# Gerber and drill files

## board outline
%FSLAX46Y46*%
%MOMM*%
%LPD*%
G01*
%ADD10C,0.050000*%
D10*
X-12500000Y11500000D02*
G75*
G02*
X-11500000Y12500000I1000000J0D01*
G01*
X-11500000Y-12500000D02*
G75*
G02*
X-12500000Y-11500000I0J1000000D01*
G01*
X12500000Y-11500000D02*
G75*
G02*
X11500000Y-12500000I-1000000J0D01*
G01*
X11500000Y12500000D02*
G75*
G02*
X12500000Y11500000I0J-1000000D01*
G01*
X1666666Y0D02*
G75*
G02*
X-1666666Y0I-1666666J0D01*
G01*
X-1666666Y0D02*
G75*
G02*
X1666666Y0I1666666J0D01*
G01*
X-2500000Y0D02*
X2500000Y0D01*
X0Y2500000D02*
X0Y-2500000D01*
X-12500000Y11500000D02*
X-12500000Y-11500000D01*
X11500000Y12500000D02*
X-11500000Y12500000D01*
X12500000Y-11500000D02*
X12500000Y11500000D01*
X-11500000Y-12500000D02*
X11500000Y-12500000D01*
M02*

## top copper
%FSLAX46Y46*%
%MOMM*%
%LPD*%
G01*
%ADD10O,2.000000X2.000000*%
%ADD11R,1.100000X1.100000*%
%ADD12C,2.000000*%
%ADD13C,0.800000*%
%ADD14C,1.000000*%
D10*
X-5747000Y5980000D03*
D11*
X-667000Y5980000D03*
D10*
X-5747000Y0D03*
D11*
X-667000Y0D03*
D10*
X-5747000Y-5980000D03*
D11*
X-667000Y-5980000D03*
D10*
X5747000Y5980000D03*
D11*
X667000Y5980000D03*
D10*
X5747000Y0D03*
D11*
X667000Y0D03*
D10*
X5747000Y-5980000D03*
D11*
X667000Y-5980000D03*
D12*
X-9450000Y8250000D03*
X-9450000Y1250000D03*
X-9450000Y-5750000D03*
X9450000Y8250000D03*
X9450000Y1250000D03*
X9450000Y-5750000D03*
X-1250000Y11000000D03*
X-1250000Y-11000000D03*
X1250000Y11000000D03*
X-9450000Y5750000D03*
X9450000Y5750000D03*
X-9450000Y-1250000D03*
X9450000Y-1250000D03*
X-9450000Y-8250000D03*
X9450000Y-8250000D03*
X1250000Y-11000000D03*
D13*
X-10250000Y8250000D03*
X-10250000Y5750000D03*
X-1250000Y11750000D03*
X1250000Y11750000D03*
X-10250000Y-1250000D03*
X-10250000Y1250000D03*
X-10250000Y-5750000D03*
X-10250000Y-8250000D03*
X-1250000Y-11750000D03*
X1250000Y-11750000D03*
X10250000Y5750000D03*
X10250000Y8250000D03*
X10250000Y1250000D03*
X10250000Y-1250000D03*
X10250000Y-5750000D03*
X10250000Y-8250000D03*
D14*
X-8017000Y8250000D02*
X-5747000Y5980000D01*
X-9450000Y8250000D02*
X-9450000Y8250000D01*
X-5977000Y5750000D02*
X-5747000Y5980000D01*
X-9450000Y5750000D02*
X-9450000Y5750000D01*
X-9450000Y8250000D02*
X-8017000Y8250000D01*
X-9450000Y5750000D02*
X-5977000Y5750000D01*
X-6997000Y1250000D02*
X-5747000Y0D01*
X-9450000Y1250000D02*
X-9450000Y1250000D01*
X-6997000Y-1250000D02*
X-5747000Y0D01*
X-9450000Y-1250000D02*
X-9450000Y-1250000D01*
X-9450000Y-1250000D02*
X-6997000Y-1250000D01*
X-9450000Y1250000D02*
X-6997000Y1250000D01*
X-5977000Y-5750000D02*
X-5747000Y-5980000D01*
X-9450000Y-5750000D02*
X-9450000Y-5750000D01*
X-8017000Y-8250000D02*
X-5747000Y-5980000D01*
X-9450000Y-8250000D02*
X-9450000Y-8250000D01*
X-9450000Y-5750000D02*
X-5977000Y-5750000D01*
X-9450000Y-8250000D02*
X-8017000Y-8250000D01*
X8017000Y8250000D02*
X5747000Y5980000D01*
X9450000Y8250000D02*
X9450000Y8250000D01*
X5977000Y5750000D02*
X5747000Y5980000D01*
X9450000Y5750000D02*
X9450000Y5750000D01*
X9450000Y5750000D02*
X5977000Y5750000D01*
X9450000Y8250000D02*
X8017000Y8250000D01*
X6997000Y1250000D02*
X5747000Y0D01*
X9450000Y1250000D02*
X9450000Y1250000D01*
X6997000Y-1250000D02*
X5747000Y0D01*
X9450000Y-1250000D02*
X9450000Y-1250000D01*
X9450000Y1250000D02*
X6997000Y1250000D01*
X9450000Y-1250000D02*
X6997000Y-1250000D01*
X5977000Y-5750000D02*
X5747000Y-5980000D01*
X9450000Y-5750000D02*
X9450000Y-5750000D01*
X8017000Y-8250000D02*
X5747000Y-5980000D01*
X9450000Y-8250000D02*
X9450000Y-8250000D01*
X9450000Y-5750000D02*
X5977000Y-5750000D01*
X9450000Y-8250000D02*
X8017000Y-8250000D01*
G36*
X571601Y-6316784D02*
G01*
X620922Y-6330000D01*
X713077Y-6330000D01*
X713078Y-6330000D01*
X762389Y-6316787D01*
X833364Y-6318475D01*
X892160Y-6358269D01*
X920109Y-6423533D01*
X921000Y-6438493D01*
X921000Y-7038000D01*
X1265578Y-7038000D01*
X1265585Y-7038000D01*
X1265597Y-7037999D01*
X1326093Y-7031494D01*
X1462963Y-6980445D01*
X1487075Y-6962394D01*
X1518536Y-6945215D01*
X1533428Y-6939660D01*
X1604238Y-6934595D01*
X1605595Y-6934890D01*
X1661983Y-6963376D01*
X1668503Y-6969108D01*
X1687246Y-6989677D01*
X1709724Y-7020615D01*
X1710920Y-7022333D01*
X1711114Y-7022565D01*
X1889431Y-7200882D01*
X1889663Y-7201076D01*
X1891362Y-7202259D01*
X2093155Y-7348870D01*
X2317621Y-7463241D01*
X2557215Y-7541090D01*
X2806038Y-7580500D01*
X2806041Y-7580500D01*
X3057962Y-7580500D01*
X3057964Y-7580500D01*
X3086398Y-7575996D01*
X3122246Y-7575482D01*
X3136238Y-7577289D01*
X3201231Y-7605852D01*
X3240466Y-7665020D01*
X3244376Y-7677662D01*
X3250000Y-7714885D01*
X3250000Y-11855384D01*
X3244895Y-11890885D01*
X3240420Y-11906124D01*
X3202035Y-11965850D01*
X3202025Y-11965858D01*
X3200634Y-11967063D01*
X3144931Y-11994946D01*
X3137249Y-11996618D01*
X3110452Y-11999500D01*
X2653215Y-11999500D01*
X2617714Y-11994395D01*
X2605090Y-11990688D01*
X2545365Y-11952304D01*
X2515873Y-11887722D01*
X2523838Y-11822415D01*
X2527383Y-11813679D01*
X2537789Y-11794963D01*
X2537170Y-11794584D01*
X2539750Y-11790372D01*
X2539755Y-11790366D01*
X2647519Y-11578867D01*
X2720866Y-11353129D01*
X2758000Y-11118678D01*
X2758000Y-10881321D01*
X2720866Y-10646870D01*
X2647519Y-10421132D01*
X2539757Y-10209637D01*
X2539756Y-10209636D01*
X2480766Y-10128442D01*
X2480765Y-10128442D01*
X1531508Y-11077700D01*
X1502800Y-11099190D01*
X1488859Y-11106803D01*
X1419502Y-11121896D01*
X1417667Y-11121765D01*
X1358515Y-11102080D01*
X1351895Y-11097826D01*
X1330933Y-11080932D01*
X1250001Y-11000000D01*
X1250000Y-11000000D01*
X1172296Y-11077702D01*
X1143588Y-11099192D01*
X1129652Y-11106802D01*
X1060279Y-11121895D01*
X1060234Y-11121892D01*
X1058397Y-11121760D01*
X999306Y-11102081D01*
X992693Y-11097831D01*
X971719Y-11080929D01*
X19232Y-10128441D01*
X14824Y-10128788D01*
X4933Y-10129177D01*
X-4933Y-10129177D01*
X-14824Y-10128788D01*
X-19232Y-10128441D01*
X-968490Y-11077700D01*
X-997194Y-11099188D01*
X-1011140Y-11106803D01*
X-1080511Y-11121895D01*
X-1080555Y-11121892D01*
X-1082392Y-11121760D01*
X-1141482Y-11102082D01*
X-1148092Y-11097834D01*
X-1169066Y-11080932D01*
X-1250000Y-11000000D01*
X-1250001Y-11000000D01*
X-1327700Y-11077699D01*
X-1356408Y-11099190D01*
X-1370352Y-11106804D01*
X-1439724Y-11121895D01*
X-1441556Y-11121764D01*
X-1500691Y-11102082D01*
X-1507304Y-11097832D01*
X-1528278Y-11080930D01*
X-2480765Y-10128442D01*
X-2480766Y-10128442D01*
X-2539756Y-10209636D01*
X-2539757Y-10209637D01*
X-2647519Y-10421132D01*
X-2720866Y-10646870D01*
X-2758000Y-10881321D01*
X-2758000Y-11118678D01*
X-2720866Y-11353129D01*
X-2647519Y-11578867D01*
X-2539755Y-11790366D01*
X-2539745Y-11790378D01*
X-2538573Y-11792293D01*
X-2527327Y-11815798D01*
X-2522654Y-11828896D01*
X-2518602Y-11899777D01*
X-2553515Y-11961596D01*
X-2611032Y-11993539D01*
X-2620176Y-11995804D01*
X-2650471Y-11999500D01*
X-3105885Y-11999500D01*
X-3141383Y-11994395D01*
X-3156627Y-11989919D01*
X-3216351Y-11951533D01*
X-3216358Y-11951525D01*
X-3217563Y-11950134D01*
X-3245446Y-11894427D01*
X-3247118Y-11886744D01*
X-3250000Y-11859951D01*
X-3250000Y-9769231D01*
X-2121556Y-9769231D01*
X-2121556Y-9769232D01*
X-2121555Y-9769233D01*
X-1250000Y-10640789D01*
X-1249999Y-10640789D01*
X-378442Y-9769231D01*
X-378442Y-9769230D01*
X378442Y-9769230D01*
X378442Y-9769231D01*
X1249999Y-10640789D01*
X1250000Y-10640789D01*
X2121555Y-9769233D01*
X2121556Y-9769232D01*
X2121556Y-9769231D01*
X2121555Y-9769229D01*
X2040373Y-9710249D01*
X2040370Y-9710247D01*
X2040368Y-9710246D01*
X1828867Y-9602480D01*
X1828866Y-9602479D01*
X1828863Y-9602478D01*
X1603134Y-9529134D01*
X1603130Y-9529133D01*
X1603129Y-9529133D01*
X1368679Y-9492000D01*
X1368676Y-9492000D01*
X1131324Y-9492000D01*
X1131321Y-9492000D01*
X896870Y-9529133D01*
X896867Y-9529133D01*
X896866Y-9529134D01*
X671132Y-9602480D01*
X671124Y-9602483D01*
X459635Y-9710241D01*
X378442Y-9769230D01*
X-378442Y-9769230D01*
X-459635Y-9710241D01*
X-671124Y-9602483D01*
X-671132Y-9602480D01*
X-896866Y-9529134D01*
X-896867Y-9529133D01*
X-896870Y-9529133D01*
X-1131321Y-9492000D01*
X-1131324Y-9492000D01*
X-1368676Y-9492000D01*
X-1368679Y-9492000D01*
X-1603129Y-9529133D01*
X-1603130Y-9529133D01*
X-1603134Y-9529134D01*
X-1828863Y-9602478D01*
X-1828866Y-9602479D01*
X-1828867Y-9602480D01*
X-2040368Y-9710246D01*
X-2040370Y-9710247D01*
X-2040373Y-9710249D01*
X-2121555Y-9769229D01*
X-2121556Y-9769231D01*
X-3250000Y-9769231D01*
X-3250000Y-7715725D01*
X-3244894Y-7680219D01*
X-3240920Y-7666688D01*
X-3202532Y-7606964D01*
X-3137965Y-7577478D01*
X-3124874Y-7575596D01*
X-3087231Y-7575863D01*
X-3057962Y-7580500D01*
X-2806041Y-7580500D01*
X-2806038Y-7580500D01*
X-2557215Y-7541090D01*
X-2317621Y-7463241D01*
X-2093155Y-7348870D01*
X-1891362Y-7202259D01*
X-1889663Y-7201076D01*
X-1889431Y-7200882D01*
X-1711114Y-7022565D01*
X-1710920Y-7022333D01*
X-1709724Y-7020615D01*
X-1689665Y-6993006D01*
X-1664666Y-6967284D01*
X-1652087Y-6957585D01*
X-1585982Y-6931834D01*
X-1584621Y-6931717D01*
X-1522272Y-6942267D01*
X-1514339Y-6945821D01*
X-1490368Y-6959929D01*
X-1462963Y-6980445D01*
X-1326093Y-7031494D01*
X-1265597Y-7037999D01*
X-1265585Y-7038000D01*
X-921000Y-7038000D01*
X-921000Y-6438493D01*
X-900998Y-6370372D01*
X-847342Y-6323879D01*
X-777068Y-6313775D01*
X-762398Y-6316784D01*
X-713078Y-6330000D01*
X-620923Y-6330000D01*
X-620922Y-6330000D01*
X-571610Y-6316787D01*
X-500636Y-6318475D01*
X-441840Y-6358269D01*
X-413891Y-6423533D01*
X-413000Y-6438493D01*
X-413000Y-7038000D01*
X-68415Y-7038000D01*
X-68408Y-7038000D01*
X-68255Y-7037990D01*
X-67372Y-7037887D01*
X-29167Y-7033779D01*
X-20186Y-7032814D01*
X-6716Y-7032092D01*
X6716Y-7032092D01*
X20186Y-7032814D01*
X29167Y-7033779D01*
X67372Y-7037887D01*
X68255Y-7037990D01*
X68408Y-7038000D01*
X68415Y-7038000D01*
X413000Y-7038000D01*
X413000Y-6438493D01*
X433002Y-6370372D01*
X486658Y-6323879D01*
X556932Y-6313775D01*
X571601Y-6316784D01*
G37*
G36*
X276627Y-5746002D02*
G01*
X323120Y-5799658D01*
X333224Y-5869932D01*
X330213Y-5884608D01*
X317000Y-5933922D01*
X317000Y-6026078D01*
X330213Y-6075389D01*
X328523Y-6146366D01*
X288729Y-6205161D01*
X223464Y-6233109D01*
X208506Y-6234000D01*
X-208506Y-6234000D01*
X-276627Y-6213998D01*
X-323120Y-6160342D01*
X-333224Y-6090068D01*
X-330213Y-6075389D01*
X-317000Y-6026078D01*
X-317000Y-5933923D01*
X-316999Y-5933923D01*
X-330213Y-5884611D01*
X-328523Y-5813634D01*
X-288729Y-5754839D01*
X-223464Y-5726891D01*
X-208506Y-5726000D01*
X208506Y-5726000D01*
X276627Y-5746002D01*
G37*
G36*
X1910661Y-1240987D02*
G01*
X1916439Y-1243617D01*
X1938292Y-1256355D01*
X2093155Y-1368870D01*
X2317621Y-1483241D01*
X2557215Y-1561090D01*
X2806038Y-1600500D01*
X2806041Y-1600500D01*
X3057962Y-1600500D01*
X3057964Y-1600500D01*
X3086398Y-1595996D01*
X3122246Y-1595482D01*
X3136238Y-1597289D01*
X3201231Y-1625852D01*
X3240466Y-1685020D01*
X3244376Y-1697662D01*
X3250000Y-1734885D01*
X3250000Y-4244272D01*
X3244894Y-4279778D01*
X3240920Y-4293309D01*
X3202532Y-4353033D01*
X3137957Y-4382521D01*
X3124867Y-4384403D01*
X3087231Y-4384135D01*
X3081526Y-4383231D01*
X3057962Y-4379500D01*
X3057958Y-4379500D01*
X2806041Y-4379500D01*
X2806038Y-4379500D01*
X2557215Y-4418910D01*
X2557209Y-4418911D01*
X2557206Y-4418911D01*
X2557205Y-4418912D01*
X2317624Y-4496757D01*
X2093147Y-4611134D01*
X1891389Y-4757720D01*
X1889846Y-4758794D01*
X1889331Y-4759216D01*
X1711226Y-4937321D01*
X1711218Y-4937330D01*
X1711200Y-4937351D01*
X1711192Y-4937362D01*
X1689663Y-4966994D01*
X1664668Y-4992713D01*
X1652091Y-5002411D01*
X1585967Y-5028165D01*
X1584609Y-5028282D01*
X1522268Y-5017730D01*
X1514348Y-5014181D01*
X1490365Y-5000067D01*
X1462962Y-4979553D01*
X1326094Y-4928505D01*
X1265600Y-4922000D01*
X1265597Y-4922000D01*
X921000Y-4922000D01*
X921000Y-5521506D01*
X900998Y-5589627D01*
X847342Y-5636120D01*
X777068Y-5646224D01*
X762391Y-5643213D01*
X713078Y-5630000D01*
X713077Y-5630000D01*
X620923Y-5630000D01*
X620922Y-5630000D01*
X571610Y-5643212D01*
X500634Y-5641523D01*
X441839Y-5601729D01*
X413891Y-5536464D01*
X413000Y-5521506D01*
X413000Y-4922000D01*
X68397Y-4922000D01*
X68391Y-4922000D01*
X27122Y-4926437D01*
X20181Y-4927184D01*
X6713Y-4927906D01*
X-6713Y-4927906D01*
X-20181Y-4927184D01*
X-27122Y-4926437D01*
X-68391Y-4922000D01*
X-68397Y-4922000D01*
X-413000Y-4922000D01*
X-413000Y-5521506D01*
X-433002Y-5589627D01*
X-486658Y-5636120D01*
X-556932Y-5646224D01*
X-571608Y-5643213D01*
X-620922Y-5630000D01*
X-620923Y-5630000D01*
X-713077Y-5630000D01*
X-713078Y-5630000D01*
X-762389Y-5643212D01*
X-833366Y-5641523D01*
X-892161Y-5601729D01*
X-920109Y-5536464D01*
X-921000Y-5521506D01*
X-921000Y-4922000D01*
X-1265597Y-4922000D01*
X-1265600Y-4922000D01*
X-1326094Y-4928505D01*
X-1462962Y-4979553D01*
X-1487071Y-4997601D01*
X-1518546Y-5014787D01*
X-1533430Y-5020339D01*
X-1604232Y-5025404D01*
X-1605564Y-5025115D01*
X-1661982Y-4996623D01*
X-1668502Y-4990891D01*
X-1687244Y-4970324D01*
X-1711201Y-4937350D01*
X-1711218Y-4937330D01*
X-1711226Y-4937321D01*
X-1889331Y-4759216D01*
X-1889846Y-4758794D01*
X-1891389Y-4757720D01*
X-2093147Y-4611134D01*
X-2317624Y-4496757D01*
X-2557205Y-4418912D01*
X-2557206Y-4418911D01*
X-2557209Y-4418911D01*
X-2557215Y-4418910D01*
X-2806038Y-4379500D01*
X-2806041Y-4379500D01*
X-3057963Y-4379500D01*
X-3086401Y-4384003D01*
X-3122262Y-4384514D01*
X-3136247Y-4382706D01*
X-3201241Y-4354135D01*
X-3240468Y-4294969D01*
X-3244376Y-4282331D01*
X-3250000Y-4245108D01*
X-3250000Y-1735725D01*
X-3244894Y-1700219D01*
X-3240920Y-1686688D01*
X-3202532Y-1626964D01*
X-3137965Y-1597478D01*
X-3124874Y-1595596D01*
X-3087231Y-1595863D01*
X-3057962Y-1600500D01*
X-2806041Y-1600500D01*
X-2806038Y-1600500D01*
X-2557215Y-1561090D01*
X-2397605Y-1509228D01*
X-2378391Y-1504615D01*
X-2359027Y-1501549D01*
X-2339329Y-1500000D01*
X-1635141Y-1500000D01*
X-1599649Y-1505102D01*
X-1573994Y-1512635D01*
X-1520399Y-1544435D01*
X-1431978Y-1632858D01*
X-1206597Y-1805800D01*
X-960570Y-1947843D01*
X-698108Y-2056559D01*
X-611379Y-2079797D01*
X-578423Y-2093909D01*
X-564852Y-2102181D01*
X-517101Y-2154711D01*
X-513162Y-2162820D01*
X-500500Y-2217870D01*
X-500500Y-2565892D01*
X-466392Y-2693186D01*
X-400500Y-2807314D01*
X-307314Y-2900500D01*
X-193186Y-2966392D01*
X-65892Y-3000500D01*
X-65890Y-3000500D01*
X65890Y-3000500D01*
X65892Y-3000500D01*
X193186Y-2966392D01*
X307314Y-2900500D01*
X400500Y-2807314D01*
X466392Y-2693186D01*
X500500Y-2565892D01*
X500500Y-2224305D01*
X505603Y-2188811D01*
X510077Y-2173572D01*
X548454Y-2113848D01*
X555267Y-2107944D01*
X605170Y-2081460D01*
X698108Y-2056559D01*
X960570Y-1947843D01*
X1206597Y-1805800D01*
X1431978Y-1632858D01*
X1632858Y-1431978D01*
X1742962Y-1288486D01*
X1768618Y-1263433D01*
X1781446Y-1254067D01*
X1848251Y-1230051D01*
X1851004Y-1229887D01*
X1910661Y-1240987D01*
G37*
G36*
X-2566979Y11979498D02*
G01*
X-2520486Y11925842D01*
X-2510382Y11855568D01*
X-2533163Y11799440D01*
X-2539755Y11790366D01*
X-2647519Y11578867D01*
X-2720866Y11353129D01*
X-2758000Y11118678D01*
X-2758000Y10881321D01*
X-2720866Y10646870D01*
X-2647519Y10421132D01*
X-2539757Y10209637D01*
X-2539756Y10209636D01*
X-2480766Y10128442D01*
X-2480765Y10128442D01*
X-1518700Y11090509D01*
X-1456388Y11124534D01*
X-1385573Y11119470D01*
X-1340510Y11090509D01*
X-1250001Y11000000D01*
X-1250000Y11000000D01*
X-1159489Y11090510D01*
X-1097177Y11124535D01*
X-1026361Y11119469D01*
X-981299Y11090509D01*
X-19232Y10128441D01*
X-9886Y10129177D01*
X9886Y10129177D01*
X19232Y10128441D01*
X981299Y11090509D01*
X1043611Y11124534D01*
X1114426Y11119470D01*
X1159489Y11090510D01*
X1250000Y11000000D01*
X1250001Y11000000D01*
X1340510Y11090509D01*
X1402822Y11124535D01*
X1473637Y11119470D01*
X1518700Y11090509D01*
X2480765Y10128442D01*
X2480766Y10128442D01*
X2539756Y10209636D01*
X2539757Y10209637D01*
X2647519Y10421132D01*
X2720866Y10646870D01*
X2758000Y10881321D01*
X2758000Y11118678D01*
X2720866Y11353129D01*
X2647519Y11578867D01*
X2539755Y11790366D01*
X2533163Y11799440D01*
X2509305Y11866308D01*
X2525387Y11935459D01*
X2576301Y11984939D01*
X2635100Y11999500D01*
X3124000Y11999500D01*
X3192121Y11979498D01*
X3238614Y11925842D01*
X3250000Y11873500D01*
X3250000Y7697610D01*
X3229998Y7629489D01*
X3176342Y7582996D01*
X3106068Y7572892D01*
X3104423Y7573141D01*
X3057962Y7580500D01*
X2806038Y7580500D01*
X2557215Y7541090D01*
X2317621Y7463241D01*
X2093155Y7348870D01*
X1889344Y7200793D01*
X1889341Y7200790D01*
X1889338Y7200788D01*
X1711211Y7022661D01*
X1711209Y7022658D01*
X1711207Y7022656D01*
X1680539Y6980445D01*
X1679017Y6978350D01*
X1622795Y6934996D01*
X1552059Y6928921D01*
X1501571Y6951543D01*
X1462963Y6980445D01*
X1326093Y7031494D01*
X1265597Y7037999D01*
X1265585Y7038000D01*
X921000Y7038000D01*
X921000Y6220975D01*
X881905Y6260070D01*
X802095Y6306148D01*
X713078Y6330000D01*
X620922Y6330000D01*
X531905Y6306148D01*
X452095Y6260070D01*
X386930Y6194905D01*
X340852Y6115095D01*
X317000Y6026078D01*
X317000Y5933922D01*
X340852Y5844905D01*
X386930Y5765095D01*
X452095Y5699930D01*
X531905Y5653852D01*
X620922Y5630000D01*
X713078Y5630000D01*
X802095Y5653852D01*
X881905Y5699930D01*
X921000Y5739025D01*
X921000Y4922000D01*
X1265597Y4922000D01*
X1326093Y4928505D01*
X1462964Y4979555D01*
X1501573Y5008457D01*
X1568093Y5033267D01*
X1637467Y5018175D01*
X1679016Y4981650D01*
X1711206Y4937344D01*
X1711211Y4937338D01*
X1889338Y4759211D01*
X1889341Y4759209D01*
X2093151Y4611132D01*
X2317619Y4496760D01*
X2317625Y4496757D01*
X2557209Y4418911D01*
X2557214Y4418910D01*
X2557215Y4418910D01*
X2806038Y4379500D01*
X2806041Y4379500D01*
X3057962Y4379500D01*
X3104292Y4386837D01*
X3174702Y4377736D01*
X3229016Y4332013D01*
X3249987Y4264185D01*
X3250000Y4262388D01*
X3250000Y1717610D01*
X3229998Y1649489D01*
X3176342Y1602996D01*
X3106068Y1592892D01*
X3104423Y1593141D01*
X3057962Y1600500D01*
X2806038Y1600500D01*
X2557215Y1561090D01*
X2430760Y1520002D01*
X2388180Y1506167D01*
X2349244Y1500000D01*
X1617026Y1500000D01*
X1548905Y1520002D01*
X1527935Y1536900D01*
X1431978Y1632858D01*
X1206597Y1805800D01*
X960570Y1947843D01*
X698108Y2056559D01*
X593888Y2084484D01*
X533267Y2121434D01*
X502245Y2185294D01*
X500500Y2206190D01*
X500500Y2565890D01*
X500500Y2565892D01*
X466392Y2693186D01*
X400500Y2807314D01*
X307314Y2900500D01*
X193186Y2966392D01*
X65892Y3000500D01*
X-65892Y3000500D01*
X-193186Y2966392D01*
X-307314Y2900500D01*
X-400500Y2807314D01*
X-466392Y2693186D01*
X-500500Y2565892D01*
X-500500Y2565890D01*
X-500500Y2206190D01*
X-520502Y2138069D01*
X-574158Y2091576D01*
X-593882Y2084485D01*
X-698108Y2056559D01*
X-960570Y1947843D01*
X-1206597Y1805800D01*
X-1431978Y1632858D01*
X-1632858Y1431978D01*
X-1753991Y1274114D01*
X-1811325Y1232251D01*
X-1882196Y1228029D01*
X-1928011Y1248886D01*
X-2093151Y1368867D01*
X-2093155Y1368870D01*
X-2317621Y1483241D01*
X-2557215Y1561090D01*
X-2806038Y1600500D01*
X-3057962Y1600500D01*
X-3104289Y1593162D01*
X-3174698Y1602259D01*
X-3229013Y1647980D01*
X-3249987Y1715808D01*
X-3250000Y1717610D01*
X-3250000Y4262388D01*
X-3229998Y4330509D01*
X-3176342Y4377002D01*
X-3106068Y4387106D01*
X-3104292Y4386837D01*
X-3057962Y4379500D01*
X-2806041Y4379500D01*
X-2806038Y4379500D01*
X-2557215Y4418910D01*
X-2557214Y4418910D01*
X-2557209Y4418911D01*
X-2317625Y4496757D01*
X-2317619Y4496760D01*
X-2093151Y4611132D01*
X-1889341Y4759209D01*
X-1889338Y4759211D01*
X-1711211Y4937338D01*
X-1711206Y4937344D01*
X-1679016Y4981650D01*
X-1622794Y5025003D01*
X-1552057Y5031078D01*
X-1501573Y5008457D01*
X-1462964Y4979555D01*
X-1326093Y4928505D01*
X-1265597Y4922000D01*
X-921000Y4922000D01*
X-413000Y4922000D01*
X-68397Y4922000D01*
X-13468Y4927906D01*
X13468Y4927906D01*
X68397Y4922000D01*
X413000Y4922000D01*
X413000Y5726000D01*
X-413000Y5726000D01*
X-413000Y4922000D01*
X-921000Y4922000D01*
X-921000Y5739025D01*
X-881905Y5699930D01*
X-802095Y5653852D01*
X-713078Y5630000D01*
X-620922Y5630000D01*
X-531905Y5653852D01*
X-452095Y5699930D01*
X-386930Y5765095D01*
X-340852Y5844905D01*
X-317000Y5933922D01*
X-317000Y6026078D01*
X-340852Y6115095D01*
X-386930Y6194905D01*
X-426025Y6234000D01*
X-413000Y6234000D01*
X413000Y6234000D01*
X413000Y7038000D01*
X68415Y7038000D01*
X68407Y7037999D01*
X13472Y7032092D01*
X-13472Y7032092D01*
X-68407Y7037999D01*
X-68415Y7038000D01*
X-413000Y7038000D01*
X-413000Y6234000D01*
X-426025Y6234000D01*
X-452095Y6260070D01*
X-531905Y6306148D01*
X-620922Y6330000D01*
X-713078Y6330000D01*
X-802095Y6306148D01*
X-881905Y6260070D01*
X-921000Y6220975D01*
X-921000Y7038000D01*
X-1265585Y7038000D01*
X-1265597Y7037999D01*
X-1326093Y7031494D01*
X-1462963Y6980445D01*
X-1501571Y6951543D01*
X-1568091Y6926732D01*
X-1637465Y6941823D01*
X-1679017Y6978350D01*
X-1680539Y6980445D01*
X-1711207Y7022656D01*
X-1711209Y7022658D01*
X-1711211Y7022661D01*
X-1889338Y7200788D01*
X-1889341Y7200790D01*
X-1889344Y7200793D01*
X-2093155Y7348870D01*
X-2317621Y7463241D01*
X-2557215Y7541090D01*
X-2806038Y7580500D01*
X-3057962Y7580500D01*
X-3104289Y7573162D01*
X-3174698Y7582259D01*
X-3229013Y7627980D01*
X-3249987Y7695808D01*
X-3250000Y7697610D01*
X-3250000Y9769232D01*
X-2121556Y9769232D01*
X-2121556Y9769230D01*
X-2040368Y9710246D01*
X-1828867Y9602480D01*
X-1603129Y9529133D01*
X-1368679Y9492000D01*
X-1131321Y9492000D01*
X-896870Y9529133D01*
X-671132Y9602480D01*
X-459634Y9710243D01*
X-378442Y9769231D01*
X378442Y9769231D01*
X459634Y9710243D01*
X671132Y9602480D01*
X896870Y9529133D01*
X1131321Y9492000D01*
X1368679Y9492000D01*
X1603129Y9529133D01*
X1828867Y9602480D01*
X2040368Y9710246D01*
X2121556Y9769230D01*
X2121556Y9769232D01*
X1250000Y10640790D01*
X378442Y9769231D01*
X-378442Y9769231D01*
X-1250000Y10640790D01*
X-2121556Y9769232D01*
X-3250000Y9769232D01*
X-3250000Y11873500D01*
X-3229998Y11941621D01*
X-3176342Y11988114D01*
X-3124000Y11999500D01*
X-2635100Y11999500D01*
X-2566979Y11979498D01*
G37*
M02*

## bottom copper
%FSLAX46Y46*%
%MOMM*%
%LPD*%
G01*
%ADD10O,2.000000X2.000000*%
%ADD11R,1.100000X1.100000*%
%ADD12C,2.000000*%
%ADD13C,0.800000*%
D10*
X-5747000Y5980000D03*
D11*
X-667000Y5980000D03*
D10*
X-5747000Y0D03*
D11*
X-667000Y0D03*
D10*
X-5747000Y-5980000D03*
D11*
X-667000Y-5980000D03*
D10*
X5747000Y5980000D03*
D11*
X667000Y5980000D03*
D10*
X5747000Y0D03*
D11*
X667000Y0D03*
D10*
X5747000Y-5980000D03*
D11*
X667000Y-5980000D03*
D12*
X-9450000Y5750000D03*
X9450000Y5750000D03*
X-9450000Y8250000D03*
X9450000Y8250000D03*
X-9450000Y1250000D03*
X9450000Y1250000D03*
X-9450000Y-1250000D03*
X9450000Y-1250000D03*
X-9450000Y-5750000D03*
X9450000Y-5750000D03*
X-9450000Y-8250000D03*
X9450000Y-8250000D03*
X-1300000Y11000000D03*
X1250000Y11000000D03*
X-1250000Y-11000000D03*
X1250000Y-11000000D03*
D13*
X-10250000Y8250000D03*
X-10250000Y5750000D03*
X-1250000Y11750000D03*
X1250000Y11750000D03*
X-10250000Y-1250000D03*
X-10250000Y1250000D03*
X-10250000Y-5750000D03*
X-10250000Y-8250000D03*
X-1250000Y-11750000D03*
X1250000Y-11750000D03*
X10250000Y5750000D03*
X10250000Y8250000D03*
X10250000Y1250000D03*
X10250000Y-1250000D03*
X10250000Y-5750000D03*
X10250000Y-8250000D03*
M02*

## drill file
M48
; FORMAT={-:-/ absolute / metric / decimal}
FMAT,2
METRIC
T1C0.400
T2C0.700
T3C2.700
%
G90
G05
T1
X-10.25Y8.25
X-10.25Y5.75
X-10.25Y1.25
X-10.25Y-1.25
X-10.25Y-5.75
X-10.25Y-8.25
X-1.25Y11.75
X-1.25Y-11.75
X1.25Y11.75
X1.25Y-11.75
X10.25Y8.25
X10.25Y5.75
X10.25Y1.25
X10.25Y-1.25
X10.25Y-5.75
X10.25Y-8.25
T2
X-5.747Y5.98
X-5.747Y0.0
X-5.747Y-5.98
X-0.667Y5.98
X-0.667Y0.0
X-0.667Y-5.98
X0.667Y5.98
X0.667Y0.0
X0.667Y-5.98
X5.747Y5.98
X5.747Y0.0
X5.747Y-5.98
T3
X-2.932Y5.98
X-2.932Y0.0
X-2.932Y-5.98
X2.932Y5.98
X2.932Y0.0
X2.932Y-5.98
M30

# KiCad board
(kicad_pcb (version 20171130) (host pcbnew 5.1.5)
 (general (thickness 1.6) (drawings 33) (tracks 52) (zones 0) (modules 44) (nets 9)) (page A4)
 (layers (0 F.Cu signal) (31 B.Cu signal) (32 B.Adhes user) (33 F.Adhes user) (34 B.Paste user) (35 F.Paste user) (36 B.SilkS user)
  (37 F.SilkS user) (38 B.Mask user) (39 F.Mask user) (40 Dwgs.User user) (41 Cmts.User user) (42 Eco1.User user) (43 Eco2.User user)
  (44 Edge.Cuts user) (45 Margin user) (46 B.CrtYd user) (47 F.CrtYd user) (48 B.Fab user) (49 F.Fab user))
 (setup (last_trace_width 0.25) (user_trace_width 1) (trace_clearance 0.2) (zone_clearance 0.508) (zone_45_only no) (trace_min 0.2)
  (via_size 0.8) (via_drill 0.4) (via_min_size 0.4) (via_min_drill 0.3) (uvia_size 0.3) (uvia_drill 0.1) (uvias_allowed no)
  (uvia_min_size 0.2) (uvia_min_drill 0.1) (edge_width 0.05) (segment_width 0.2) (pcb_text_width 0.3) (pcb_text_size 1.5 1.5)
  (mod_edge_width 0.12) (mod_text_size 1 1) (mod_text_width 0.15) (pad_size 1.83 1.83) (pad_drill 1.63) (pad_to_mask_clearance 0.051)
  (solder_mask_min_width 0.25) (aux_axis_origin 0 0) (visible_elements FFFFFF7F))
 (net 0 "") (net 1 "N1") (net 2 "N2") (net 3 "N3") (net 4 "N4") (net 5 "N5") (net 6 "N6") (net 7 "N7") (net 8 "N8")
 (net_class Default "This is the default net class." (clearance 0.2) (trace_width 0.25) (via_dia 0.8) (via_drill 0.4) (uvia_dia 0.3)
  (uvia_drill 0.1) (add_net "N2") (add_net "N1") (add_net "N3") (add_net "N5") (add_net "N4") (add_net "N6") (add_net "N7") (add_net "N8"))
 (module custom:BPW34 (layer F.Cu) (at -2.932 -5.98 180)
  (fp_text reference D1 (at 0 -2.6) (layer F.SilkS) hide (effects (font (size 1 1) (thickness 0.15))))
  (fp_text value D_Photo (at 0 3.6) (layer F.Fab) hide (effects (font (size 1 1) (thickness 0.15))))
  (pad 2 thru_hole oval (at 2.815 0 180) (size 2 2) (drill 0.7) (layers *.Cu *.Mask) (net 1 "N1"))
  (pad 1 thru_hole rect (at -2.265 0 180) (size 1.1 1.1) (drill 0.7) (layers *.Cu *.Mask) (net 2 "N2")))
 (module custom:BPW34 (layer F.Cu) (at -2.932 0 180)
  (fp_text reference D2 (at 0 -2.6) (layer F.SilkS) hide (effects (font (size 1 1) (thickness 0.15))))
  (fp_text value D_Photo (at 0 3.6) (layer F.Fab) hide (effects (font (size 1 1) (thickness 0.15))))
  (pad 2 thru_hole oval (at 2.815 0 180) (size 2 2) (drill 0.7) (layers *.Cu *.Mask) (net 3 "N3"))
  (pad 1 thru_hole rect (at -2.265 0 180) (size 1.1 1.1) (drill 0.7) (layers *.Cu *.Mask) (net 2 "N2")))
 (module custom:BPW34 (layer F.Cu) (at -2.932 5.98 180)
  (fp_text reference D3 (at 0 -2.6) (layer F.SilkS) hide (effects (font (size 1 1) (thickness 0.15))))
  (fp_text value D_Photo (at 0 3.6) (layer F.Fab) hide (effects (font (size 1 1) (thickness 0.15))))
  (pad 2 thru_hole oval (at 2.815 0 180) (size 2 2) (drill 0.7) (layers *.Cu *.Mask) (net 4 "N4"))
  (pad 1 thru_hole rect (at -2.265 0 180) (size 1.1 1.1) (drill 0.7) (layers *.Cu *.Mask) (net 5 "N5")))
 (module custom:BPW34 (layer F.Cu) (at 2.932 -5.98)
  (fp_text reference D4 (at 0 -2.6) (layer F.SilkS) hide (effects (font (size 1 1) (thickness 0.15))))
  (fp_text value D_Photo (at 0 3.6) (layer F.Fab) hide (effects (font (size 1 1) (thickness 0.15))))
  (pad 2 thru_hole oval (at 2.815 0) (size 2 2) (drill 0.7) (layers *.Cu *.Mask) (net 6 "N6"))
  (pad 1 thru_hole rect (at -2.265 0) (size 1.1 1.1) (drill 0.7) (layers *.Cu *.Mask) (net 2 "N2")))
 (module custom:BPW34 (layer F.Cu) (at 2.932 0)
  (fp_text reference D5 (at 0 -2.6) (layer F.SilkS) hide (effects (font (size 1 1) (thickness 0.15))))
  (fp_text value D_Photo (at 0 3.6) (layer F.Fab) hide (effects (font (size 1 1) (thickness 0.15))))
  (pad 2 thru_hole oval (at 2.815 0) (size 2 2) (drill 0.7) (layers *.Cu *.Mask) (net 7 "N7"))
  (pad 1 thru_hole rect (at -2.265 0) (size 1.1 1.1) (drill 0.7) (layers *.Cu *.Mask) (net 5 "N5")))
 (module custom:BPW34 (layer F.Cu) (at 2.932 5.98)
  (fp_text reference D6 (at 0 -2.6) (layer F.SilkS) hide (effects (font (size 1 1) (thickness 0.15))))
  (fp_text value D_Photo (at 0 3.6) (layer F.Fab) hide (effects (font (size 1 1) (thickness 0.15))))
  (pad 2 thru_hole oval (at 2.815 0) (size 2 2) (drill 0.7) (layers *.Cu *.Mask) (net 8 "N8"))
  (pad 1 thru_hole rect (at -2.265 0) (size 1.1 1.1) (drill 0.7) (layers *.Cu *.Mask) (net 5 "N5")))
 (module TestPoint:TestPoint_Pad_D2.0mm (layer F.Cu) (at -9.45 -8.25)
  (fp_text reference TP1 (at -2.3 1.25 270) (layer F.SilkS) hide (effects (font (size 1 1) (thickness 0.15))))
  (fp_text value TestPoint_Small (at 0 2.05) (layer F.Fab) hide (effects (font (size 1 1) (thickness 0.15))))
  (pad 1 smd circle (at 0 0) (size 2 2) (layers F.Cu F.Mask) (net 1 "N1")))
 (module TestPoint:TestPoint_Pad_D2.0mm (layer F.Cu) (at -9.45 -1.25)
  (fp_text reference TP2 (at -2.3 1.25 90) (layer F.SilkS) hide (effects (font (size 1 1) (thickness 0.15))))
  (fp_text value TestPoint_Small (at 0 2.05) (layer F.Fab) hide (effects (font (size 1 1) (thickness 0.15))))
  (pad 1 smd circle (at 0 0) (size 2 2) (layers F.Cu F.Mask) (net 3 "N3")))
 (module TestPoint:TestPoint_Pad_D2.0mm (layer F.Cu) (at -9.45 5.75)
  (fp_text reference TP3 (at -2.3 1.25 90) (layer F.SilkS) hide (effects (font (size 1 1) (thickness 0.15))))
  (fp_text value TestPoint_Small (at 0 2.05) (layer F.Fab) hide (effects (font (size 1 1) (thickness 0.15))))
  (pad 1 smd circle (at 0 0) (size 2 2) (layers F.Cu F.Mask) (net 4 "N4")))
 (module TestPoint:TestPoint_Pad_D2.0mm (layer F.Cu) (at 9.45 -8.25)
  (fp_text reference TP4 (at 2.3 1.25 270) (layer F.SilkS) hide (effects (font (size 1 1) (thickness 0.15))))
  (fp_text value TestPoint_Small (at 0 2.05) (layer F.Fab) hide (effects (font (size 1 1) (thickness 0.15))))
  (pad 1 smd circle (at 0 0) (size 2 2) (layers F.Cu F.Mask) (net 6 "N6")))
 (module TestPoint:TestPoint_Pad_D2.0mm (layer F.Cu) (at 9.45 -1.25)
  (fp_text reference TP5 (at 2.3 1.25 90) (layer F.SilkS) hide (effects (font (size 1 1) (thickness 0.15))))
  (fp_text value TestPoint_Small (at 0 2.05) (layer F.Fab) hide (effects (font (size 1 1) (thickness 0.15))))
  (pad 1 smd circle (at 0 0) (size 2 2) (layers F.Cu F.Mask) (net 7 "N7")))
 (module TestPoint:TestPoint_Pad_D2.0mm (layer F.Cu) (at 9.45 5.75)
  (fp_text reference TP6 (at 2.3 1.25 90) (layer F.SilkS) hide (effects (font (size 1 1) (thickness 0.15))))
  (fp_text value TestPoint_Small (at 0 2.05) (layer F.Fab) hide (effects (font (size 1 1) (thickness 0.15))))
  (pad 1 smd circle (at 0 0) (size 2 2) (layers F.Cu F.Mask) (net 8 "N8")))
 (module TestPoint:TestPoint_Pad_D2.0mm (layer F.Cu) (at -1.25 -11)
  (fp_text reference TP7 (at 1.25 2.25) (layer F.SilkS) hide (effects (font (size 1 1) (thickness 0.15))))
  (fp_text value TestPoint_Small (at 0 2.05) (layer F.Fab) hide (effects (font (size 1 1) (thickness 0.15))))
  (pad 1 smd circle (at 0 0) (size 2 2) (layers F.Cu F.Mask) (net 2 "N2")))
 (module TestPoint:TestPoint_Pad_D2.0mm (layer F.Cu) (at -1.25 11)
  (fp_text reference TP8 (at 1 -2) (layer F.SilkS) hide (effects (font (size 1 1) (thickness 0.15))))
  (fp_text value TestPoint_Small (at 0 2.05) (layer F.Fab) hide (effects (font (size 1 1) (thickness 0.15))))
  (pad 1 smd circle (at 0 0) (size 2 2) (layers F.Cu F.Mask) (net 5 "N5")))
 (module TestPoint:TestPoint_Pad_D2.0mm (layer F.Cu) (at 1.25 -11)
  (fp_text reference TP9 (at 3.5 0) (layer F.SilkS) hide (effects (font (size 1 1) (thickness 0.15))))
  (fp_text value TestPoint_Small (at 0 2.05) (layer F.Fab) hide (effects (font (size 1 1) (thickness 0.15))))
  (pad 1 smd circle (at 0 0) (size 2 2) (layers F.Cu F.Mask) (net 2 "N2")))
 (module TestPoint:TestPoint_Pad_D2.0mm (layer F.Cu) (at -9.45 -5.75)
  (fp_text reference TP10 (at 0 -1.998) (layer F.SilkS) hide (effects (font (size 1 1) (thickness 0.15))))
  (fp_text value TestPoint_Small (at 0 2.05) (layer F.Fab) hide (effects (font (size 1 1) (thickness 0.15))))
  (pad 1 smd circle (at 0 0) (size 2 2) (layers F.Cu F.Mask) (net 1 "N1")))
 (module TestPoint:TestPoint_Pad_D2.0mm (layer F.Cu) (at 9.45 -5.75)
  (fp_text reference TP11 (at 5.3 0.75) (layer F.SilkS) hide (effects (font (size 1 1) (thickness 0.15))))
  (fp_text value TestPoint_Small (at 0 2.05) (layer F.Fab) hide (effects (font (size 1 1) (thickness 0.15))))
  (pad 1 smd circle (at 0 0) (size 2 2) (layers F.Cu F.Mask) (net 6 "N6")))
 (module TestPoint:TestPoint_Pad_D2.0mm (layer F.Cu) (at -9.45 1.25)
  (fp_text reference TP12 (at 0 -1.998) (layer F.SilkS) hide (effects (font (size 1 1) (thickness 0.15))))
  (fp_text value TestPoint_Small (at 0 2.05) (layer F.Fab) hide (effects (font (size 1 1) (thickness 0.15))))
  (pad 1 smd circle (at 0 0) (size 2 2) (layers F.Cu F.Mask) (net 3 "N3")))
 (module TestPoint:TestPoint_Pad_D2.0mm (layer F.Cu) (at 9.45 1.25)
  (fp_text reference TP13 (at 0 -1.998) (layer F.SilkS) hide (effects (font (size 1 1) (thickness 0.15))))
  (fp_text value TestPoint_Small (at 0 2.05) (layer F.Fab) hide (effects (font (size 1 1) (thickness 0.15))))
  (pad 1 smd circle (at 0 0) (size 2 2) (layers F.Cu F.Mask) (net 7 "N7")))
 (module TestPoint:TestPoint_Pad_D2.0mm (layer F.Cu) (at -9.45 8.25)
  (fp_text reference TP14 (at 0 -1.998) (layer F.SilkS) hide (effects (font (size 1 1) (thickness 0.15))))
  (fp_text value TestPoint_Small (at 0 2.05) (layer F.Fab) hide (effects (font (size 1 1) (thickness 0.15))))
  (pad 1 smd circle (at 0 0) (size 2 2) (layers F.Cu F.Mask) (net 4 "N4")))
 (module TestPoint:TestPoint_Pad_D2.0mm (layer F.Cu) (at 9.45 8.25)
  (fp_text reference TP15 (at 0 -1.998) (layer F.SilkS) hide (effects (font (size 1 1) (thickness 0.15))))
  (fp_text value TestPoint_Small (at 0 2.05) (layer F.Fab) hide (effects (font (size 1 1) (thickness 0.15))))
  (pad 1 smd circle (at 0 0) (size 2 2) (layers F.Cu F.Mask) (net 8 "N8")))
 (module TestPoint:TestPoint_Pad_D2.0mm (layer F.Cu) (at 1.25 11)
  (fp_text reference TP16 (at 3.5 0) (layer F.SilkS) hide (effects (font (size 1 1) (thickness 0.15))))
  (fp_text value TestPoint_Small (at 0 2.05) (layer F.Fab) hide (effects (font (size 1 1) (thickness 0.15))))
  (pad 1 smd circle (at 0 0) (size 2 2) (layers F.Cu F.Mask) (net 5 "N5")))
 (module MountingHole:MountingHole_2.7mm (layer F.Cu) (at -2.932 -5.98)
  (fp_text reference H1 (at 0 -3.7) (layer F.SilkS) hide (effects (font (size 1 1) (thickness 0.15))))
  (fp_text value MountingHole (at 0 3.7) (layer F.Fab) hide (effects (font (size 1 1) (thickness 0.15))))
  (pad 1 np_thru_hole circle (at 0 0) (size 2.7 2.7) (drill 2.7) (layers *.Cu *.Mask)))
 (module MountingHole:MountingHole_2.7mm (layer F.Cu) (at -2.932 0)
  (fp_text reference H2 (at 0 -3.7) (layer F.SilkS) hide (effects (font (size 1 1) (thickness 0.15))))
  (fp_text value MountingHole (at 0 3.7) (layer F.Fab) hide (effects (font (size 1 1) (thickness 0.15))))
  (pad 1 np_thru_hole circle (at 0 0) (size 2.7 2.7) (drill 2.7) (layers *.Cu *.Mask)))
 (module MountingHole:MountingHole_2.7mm (layer F.Cu) (at -2.932 5.98)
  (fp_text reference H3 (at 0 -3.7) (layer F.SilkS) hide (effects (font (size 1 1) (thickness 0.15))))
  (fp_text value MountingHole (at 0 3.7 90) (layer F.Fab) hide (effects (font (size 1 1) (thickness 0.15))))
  (pad 1 np_thru_hole circle (at 0 0) (size 2.7 2.7) (drill 2.7) (layers *.Cu *.Mask)))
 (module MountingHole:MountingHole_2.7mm (layer F.Cu) (at 2.932 -5.98)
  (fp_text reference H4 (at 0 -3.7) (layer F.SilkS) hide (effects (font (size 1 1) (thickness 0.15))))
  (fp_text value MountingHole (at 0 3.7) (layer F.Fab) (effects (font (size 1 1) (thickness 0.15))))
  (pad 1 np_thru_hole circle (at 0 0) (size 2.7 2.7) (drill 2.7) (layers *.Cu *.Mask)))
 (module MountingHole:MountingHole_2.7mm (layer F.Cu) (at 2.932 0)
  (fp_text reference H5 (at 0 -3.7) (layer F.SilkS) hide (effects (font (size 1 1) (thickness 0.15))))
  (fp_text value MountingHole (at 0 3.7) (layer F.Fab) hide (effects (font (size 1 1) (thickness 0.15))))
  (pad 1 np_thru_hole circle (at 0 0) (size 2.7 2.7) (drill 2.7) (layers *.Cu *.Mask)))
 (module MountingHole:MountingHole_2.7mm (layer F.Cu) (at 2.932 5.98)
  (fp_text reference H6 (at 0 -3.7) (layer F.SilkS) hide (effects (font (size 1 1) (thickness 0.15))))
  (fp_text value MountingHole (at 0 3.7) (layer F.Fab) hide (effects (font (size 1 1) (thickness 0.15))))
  (pad 1 np_thru_hole circle (at 0 0) (size 2.7 2.7) (drill 2.7) (layers *.Cu *.Mask)))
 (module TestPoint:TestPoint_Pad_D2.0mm (layer B.Cu) (at -9.45 -5.75)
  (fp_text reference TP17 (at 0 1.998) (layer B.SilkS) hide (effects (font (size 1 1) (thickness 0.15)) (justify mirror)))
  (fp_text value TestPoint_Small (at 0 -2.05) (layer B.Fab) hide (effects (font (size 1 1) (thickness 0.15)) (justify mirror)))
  (pad 1 smd circle (at 0 0) (size 2 2) (layers B.Cu B.Mask) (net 1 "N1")))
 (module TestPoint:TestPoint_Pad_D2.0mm (layer B.Cu) (at 9.45 -5.75)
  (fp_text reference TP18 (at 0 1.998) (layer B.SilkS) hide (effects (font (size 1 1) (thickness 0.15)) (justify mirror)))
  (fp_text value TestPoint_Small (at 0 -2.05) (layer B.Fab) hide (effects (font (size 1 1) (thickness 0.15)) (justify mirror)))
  (pad 1 smd circle (at 0 0) (size 2 2) (layers B.Cu B.Mask) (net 6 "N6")))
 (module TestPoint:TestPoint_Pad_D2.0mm (layer B.Cu) (at -9.45 -8.25)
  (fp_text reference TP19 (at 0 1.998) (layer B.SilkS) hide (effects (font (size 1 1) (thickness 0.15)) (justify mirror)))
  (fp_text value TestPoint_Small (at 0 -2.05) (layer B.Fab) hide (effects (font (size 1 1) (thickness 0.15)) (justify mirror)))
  (pad 1 smd circle (at 0 0) (size 2 2) (layers B.Cu B.Mask) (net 1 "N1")))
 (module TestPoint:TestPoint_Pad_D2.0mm (layer B.Cu) (at 9.45 -8.25)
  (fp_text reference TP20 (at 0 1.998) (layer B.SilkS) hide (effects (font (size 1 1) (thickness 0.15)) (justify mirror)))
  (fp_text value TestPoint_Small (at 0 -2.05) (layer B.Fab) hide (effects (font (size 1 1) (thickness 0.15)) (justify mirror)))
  (pad 1 smd circle (at 0 0) (size 2 2) (layers B.Cu B.Mask) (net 6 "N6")))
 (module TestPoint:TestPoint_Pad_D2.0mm (layer B.Cu) (at -9.45 -1.25)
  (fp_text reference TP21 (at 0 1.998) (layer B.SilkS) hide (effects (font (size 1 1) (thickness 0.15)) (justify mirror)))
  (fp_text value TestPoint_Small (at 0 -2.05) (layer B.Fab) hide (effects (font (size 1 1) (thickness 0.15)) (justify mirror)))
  (pad 1 smd circle (at 0 0) (size 2 2) (layers B.Cu B.Mask) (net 3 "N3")))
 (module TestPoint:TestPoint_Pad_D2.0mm (layer B.Cu) (at 9.45 -1.25)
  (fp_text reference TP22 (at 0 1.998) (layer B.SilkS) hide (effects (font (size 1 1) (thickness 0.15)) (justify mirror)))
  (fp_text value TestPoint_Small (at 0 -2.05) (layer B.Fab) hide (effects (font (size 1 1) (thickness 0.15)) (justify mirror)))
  (pad 1 smd circle (at 0 0) (size 2 2) (layers B.Cu B.Mask) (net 7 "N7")))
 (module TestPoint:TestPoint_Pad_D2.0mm (layer B.Cu) (at -9.45 1.25)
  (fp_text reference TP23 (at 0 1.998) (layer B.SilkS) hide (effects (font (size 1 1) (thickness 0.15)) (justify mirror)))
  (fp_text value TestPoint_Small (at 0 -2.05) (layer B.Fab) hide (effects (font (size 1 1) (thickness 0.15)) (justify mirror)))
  (pad 1 smd circle (at 0 0) (size 2 2) (layers B.Cu B.Mask) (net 3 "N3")))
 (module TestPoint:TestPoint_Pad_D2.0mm (layer B.Cu) (at 9.45 1.25)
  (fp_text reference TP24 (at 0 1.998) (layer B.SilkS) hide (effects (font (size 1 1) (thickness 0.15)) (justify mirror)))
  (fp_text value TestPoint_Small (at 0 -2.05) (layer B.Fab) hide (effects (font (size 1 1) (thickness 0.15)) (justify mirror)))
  (pad 1 smd circle (at 0 0) (size 2 2) (layers B.Cu B.Mask) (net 7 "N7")))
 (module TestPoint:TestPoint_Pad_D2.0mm (layer B.Cu) (at -9.45 5.75)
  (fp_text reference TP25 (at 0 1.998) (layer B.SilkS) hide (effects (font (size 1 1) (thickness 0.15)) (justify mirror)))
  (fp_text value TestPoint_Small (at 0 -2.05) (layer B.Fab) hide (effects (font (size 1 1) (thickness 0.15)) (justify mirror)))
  (pad 1 smd circle (at 0 0) (size 2 2) (layers B.Cu B.Mask) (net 4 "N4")))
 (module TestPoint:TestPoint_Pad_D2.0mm (layer B.Cu) (at 9.45 5.75)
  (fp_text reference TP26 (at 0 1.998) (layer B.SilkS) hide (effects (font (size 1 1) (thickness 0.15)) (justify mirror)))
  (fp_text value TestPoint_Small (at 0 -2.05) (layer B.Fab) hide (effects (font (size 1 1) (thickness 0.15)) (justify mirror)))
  (pad 1 smd circle (at 0 0) (size 2 2) (layers B.Cu B.Mask) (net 8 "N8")))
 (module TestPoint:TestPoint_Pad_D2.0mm (layer B.Cu) (at -9.45 8.25)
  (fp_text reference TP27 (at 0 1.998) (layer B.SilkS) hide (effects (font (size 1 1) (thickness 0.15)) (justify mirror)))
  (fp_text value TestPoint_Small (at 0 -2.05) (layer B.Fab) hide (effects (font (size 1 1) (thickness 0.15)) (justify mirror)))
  (pad 1 smd circle (at 0 0) (size 2 2) (layers B.Cu B.Mask) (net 4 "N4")))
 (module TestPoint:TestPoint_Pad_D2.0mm (layer B.Cu) (at 9.45 8.25)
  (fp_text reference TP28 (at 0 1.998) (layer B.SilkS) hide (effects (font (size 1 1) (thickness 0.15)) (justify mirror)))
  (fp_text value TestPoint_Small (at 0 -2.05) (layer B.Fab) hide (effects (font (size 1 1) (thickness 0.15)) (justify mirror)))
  (pad 1 smd circle (at 0 0) (size 2 2) (layers B.Cu B.Mask) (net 8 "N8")))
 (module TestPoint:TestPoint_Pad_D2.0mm (layer B.Cu) (at -1.3 -11)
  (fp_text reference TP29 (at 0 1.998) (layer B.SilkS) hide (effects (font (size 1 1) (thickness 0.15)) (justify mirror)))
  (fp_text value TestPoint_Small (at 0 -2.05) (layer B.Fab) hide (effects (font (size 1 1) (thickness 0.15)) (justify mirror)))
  (pad 1 smd circle (at 0 0) (size 2 2) (layers B.Cu B.Mask) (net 2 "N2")))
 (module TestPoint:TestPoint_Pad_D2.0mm (layer B.Cu) (at 1.25 -11)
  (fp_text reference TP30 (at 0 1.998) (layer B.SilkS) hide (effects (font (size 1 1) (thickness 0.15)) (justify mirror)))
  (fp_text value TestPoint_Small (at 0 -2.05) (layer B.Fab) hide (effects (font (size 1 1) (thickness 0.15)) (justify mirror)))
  (pad 1 smd circle (at 0 0) (size 2 2) (layers B.Cu B.Mask) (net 2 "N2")))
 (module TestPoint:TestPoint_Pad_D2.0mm (layer B.Cu) (at -1.25 11)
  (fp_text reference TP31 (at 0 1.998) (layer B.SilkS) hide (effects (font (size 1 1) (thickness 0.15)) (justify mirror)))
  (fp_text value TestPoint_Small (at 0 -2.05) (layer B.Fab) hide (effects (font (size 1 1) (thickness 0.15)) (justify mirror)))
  (pad 1 smd circle (at 0 0) (size 2 2) (layers B.Cu B.Mask) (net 5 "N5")))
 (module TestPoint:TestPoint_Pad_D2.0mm (layer B.Cu) (at 1.25 11)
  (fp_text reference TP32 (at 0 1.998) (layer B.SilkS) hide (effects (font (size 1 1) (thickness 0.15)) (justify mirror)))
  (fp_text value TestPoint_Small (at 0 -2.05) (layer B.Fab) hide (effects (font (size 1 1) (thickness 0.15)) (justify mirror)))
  (pad 1 smd circle (at 0 0) (size 2 2) (layers B.Cu B.Mask) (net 5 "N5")))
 (gr_arc (start -11.5 -11.5) (end -11.5 -12.5) (angle -90) (layer Edge.Cuts) (width 0.05))
 (gr_arc (start -11.5 11.5) (end -12.5 11.5) (angle -90) (layer Edge.Cuts) (width 0.05))
 (gr_arc (start 11.5 11.5) (end 11.5 12.5) (angle -90) (layer Edge.Cuts) (width 0.05))
 (gr_arc (start 11.5 -11.5) (end 12.5 -11.5) (angle -90) (layer Edge.Cuts) (width 0.05))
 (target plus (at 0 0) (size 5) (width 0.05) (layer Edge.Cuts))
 (gr_line (start -12.5 -11.5) (end -12.5 11.5) (layer Edge.Cuts) (width 0.05))
 (gr_line (start 11.5 -12.5) (end -11.5 -12.5) (layer Edge.Cuts) (width 0.05))
 (gr_line (start 12.5 11.5) (end 12.5 -11.5) (layer Edge.Cuts) (width 0.05))
 (gr_line (start -11.5 12.5) (end 11.5 12.5) (layer Edge.Cuts) (width 0.05))
 (segment (start -8.017 -8.25) (end -5.747 -5.98) (width 1) (layer F.Cu) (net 1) (status 20))
 (segment (start -9.45 -8.25) (end -9.45 -8.25) (width 1) (layer F.Cu) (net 1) (status 10))
 (segment (start -5.977 -5.75) (end -5.747 -5.98) (width 1) (layer F.Cu) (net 1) (status 30))
 (segment (start -9.45 -5.75) (end -9.45 -5.75) (width 1) (layer F.Cu) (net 1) (status 30))
 (segment (start -9.45 -8.25) (end -8.017 -8.25) (width 1) (layer F.Cu) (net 1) (status 10))
 (via (at -10.25 -8.25) (size 0.8) (drill 0.4) (layers F.Cu B.Cu) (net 1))
 (segment (start -9.45 -5.75) (end -5.977 -5.75) (width 1) (layer F.Cu) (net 1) (status 30))
 (via (at -10.25 -5.75) (size 0.8) (drill 0.4) (layers F.Cu B.Cu) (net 1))
 (via (at -1.25 -11.75) (size 0.8) (drill 0.4) (layers F.Cu B.Cu) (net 2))
 (via (at 1.25 -11.75) (size 0.8) (drill 0.4) (layers F.Cu B.Cu) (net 2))
 (segment (start -6.997 -1.25) (end -5.747 0) (width 1) (layer F.Cu) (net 3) (status 20))
 (segment (start -9.45 -1.25) (end -9.45 -1.25) (width 1) (layer F.Cu) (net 3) (status 10))
 (segment (start -6.997 1.25) (end -5.747 0) (width 1) (layer F.Cu) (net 3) (status 20))
 (segment (start -9.45 1.25) (end -9.45 1.25) (width 1) (layer F.Cu) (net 3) (status 10))
 (segment (start -9.45 1.25) (end -6.997 1.25) (width 1) (layer F.Cu) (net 3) (status 10))
 (via (at -10.25 1.25) (size 0.8) (drill 0.4) (layers F.Cu B.Cu) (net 3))
 (segment (start -9.45 -1.25) (end -6.997 -1.25) (width 1) (layer F.Cu) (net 3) (status 10))
 (via (at -10.25 -1.25) (size 0.8) (drill 0.4) (layers F.Cu B.Cu) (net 3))
 (segment (start -5.977 5.75) (end -5.747 5.98) (width 1) (layer F.Cu) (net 4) (status 30))
 (segment (start -9.45 5.75) (end -9.45 5.75) (width 1) (layer F.Cu) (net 4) (status 30))
 (segment (start -8.017 8.25) (end -5.747 5.98) (width 1) (layer F.Cu) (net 4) (status 20))
 (segment (start -9.45 8.25) (end -9.45 8.25) (width 1) (layer F.Cu) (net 4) (status 10))
 (segment (start -9.45 5.75) (end -5.977 5.75) (width 1) (layer F.Cu) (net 4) (status 30))
 (via (at -10.25 5.75) (size 0.8) (drill 0.4) (layers F.Cu B.Cu) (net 4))
 (segment (start -9.45 8.25) (end -8.017 8.25) (width 1) (layer F.Cu) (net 4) (status 10))
 (via (at -10.25 8.25) (size 0.8) (drill 0.4) (layers F.Cu B.Cu) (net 4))
 (via (at -1.25 11.75) (size 0.8) (drill 0.4) (layers F.Cu B.Cu) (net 5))
 (via (at 1.25 11.75) (size 0.8) (drill 0.4) (layers F.Cu B.Cu) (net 5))
 (segment (start 8.017 -8.25) (end 5.747 -5.98) (width 1) (layer F.Cu) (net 6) (status 20))
 (segment (start 9.45 -8.25) (end 9.45 -8.25) (width 1) (layer F.Cu) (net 6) (status 10))
 (segment (start 5.977 -5.75) (end 5.747 -5.98) (width 1) (layer F.Cu) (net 6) (status 30))
 (segment (start 9.45 -5.75) (end 9.45 -5.75) (width 1) (layer F.Cu) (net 6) (status 30))
 (segment (start 9.45 -5.75) (end 5.977 -5.75) (width 1) (layer F.Cu) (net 6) (status 30))
 (via (at 10.25 -5.75) (size 0.8) (drill 0.4) (layers F.Cu B.Cu) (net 6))
 (segment (start 9.45 -8.25) (end 8.017 -8.25) (width 1) (layer F.Cu) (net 6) (status 10))
 (via (at 10.25 -8.25) (size 0.8) (drill 0.4) (layers F.Cu B.Cu) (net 6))
 (segment (start 6.997 -1.25) (end 5.747 0) (width 1) (layer F.Cu) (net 7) (status 20))
 (segment (start 9.45 -1.25) (end 9.45 -1.25) (width 1) (layer F.Cu) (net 7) (status 10))
 (segment (start 6.997 1.25) (end 5.747 0) (width 1) (layer F.Cu) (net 7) (status 20))
 (segment (start 9.45 1.25) (end 9.45 1.25) (width 1) (layer F.Cu) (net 7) (status 10))
 (segment (start 9.45 -1.25) (end 6.997 -1.25) (width 1) (layer F.Cu) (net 7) (status 10))
 (via (at 10.25 -1.25) (size 0.8) (drill 0.4) (layers F.Cu B.Cu) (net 7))
 (segment (start 9.45 1.25) (end 6.997 1.25) (width 1) (layer F.Cu) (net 7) (status 10))
 (via (at 10.25 1.25) (size 0.8) (drill 0.4) (layers F.Cu B.Cu) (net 7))
 (segment (start 5.977 5.75) (end 5.747 5.98) (width 1) (layer F.Cu) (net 8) (status 30))
 (segment (start 9.45 5.75) (end 9.45 5.75) (width 1) (layer F.Cu) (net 8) (status 30))
 (segment (start 8.017 8.25) (end 5.747 5.98) (width 1) (layer F.Cu) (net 8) (status 20))
 (segment (start 9.45 8.25) (end 9.45 8.25) (width 1) (layer F.Cu) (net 8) (status 10))
 (segment (start 9.45 5.75) (end 5.977 5.75) (width 1) (layer F.Cu) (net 8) (status 30))
 (via (at 10.25 5.75) (size 0.8) (drill 0.4) (layers F.Cu B.Cu) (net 8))
 (segment (start 9.45 8.25) (end 8.017 8.25) (width 1) (layer F.Cu) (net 8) (status 10))
 (via (at 10.25 8.25) (size 0.8) (drill 0.4) (layers F.Cu B.Cu) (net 8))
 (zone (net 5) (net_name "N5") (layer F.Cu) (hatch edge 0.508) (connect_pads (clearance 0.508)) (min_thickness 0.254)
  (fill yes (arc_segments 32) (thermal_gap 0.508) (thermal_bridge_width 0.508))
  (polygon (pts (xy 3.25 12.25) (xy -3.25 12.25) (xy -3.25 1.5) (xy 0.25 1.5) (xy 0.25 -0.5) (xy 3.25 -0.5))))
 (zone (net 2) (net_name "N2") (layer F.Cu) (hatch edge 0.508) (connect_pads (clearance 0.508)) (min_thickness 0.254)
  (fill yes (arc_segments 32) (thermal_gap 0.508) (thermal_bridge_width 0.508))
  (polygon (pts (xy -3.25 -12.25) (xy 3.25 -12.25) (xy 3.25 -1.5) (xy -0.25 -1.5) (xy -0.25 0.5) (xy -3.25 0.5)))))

